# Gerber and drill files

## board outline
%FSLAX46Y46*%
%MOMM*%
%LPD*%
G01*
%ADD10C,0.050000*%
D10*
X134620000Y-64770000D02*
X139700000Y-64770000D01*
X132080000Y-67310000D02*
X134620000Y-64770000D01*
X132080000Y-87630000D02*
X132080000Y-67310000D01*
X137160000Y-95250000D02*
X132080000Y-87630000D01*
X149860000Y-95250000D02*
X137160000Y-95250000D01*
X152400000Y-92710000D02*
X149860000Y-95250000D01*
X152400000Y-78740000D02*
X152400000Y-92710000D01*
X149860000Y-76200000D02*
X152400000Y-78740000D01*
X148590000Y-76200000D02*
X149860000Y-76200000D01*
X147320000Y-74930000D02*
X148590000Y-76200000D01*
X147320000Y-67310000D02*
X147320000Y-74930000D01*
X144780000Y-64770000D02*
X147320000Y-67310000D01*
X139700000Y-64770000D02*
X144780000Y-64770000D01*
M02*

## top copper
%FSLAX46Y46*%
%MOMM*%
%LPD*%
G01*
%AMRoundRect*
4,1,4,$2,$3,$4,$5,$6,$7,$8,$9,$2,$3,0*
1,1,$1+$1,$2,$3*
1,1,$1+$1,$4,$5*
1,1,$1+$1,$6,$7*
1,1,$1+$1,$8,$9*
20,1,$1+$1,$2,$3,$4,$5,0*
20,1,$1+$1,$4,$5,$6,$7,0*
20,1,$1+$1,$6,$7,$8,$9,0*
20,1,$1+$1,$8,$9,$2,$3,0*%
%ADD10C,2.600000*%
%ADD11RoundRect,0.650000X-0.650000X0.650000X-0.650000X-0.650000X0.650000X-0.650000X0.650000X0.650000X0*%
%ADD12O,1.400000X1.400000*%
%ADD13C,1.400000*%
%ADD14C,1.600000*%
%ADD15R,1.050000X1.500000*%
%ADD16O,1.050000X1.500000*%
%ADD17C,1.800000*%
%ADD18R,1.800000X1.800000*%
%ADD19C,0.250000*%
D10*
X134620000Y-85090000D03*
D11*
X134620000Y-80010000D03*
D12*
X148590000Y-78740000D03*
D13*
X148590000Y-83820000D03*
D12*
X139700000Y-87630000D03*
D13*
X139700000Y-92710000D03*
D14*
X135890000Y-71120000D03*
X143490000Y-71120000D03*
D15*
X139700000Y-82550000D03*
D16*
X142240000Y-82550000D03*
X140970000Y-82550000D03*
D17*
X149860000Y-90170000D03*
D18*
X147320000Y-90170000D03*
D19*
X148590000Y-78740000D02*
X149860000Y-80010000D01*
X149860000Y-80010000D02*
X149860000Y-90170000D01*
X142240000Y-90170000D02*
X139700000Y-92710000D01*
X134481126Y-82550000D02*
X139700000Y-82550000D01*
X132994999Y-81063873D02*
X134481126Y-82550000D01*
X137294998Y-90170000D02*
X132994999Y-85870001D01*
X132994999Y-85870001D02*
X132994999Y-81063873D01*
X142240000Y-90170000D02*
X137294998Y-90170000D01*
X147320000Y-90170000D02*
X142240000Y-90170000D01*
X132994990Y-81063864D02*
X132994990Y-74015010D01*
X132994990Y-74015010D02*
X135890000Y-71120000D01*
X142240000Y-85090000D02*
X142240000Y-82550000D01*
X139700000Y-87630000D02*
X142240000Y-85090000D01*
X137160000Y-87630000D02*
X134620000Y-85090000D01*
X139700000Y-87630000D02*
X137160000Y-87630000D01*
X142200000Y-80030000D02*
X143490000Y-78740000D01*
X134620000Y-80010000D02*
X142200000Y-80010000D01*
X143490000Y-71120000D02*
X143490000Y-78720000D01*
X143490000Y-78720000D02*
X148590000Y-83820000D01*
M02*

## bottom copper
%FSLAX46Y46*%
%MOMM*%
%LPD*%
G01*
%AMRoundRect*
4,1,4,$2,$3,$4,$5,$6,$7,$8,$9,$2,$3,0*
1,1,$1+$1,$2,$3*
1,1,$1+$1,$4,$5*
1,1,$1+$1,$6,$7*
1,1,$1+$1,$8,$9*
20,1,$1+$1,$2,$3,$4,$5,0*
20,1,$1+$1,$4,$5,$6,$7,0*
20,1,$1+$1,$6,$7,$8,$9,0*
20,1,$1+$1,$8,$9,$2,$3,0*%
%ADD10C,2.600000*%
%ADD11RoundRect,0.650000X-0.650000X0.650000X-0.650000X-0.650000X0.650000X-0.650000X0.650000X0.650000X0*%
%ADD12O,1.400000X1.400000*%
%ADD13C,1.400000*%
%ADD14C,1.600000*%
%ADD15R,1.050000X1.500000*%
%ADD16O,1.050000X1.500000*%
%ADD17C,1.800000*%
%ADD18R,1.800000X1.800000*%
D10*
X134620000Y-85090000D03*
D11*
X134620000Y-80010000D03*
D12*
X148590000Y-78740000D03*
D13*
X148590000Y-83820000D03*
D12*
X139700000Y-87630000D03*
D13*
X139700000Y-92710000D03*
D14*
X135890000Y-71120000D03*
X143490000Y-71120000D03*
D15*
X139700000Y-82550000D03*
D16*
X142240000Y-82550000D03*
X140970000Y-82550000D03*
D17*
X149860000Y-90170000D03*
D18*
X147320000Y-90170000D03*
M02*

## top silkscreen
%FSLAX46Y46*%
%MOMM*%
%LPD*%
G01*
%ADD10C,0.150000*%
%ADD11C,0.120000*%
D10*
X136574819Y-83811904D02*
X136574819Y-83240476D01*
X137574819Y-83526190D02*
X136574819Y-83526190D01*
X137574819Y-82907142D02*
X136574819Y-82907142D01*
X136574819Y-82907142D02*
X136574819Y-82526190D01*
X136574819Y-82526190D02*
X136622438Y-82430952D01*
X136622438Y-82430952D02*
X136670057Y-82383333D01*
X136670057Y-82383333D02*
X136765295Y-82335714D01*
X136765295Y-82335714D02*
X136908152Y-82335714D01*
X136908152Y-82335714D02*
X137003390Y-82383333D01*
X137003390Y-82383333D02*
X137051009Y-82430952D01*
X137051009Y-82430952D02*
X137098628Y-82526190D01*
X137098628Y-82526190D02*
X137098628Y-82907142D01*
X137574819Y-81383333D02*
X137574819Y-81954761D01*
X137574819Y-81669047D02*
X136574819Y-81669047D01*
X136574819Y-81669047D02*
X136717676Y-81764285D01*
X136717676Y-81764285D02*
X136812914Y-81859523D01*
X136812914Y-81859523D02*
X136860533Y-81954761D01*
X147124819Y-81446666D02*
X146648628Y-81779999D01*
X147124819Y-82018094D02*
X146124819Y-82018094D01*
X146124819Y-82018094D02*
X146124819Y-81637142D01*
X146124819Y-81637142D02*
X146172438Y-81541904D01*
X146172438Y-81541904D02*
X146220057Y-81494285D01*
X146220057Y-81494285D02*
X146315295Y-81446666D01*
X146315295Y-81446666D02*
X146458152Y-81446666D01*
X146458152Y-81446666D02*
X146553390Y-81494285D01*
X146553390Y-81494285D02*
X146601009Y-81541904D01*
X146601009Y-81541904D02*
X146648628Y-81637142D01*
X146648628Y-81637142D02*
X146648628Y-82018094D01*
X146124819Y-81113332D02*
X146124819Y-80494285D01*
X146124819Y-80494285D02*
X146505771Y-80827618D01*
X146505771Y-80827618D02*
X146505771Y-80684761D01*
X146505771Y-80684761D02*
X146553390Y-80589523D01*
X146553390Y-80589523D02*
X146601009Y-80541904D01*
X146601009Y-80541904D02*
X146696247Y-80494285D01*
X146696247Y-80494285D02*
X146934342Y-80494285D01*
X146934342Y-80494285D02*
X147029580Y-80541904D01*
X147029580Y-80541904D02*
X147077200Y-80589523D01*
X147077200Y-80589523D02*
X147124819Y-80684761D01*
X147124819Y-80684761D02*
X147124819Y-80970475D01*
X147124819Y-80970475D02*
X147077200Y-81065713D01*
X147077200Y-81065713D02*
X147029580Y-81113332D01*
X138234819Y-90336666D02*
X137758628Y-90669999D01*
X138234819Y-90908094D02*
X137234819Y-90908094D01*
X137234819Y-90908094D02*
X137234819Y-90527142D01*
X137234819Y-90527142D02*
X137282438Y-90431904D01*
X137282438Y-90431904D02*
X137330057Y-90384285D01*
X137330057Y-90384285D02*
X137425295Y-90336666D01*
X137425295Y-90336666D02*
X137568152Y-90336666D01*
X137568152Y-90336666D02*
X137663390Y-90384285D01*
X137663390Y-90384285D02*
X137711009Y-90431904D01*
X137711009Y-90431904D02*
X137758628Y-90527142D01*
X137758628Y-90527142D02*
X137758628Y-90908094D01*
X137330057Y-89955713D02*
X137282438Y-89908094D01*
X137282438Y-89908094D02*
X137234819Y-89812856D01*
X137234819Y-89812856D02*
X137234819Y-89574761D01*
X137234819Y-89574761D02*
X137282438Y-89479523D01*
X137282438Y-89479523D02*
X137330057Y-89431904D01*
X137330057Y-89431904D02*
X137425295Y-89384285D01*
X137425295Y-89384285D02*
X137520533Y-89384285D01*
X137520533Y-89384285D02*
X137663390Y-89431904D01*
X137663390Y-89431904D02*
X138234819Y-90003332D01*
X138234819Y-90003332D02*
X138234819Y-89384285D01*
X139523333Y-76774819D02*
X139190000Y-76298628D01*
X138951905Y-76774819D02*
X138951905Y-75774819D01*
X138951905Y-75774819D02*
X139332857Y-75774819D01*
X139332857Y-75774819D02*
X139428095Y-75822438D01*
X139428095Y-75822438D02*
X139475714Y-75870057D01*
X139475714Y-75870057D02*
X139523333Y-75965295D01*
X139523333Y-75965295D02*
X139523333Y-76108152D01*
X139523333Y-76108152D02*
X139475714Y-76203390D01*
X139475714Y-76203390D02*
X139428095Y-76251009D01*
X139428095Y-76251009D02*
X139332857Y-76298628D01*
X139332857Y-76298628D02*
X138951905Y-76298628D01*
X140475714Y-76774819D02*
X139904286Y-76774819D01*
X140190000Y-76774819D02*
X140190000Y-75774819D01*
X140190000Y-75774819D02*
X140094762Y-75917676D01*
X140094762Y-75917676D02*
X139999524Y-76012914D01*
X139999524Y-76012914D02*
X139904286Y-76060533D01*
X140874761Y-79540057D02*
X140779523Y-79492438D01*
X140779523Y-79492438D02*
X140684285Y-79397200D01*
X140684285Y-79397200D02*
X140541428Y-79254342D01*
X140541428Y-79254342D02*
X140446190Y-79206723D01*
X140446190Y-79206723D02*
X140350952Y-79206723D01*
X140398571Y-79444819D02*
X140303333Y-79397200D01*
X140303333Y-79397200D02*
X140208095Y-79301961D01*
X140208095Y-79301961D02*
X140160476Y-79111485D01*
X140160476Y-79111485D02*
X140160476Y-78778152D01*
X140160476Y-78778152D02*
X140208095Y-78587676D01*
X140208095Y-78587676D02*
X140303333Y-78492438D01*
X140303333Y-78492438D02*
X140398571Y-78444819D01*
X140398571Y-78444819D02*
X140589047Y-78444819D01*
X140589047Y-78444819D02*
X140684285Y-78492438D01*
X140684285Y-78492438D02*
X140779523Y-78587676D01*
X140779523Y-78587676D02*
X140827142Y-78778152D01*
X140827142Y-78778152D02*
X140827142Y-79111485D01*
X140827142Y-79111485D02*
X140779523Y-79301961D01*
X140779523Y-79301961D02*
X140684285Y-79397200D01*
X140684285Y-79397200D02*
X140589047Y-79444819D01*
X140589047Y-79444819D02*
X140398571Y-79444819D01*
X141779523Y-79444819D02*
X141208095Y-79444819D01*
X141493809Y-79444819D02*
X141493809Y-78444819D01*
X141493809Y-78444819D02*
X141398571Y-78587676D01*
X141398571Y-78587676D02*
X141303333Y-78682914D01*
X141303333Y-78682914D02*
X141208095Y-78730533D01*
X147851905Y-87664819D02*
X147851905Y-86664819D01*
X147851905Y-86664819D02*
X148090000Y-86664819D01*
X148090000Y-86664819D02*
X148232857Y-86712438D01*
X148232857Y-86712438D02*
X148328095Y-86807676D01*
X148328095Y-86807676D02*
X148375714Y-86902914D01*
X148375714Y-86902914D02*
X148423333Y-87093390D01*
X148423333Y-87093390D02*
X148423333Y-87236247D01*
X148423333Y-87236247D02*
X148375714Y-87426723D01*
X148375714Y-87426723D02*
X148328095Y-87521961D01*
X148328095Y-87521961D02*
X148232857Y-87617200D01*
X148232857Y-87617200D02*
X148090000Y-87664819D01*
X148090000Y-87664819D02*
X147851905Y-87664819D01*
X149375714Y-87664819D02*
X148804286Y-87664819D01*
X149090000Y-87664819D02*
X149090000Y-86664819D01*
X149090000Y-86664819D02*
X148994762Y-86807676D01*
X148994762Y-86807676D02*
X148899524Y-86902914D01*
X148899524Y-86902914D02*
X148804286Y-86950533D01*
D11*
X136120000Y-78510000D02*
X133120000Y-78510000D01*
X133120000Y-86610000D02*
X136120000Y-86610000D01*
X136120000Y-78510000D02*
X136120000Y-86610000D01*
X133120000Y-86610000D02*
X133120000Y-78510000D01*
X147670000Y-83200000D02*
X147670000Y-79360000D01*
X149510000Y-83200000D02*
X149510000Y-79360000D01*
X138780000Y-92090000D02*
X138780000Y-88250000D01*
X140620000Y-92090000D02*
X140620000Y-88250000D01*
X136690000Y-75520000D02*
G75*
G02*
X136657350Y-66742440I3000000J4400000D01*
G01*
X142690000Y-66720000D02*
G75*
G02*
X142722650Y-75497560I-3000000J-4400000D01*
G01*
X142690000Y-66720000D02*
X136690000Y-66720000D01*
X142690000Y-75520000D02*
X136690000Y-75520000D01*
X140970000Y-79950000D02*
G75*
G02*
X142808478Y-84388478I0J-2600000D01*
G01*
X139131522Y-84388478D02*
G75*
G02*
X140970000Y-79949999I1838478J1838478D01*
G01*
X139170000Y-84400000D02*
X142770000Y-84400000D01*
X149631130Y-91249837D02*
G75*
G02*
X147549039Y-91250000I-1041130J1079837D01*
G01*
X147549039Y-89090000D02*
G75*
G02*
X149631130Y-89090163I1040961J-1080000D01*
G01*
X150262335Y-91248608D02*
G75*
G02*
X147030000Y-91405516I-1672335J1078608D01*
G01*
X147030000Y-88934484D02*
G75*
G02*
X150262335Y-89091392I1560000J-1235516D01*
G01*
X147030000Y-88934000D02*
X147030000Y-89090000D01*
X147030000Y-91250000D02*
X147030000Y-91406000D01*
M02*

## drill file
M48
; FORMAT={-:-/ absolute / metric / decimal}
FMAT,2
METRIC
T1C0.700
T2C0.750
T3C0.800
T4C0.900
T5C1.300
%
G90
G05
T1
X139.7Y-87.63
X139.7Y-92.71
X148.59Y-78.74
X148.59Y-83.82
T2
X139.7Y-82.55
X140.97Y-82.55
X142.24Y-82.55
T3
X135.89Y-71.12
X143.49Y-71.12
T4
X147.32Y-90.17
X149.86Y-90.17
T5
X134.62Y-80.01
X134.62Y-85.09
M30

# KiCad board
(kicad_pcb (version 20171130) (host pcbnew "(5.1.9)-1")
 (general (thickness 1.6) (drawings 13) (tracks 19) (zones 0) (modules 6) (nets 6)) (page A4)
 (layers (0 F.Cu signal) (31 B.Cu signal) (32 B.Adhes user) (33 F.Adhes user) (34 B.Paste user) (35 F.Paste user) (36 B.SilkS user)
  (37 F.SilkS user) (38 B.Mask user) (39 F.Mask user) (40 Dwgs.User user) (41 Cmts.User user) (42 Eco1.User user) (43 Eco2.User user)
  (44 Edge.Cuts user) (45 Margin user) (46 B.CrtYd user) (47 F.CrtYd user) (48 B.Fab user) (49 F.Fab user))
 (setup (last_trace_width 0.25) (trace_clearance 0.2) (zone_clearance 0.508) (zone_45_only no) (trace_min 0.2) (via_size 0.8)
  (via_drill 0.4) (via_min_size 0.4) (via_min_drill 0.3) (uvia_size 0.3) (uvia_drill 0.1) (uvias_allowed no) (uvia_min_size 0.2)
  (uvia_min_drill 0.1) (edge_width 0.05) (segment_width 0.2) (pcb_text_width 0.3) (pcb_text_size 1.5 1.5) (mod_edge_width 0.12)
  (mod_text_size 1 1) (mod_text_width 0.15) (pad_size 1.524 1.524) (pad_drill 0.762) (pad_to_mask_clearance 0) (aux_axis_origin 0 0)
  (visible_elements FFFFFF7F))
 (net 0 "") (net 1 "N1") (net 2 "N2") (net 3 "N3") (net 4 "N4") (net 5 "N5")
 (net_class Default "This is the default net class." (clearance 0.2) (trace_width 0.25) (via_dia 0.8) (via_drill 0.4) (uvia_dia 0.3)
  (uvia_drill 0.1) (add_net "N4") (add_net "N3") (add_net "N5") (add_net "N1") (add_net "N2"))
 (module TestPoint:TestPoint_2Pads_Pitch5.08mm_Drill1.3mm (layer F.Cu) (at 134.62 80.01 270)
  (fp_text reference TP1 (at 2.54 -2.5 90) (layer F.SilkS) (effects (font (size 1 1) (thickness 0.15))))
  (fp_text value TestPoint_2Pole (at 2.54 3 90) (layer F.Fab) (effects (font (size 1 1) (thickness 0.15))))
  (fp_line (start -1.5 -1.5) (end -1.5 1.5) (layer F.SilkS) (width 0.12))
  (fp_line (start 6.6 1.5) (end 6.6 -1.5) (layer F.SilkS) (width 0.12))
  (fp_line (start -1.5 -1.5) (end 6.6 -1.5) (layer F.SilkS) (width 0.12))
  (fp_line (start 6.6 1.5) (end -1.5 1.5) (layer F.SilkS) (width 0.12))
  (pad 2 thru_hole circle (at 5.08 0 270) (size 2.6 2.6) (drill 1.3) (layers *.Cu *.Mask) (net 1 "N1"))
  (pad 1 thru_hole roundrect (at 0 0 270) (size 2.6 2.6) (drill 1.3) (layers *.Cu *.Mask) (roundrect_rratio 0.25) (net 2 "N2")))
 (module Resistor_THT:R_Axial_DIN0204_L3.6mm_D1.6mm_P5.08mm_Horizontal (layer F.Cu) (at 148.59 83.82 90)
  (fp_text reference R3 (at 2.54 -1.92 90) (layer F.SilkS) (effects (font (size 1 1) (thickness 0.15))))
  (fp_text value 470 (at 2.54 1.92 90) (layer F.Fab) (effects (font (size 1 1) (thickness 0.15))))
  (fp_line (start 0.62 -0.92) (end 4.46 -0.92) (layer F.SilkS) (width 0.12))
  (fp_line (start 0.62 0.92) (end 4.46 0.92) (layer F.SilkS) (width 0.12))
  (pad 2 thru_hole oval (at 5.08 0 90) (size 1.4 1.4) (drill 0.7) (layers *.Cu *.Mask) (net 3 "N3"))
  (pad 1 thru_hole circle (at 0 0 90) (size 1.4 1.4) (drill 0.7) (layers *.Cu *.Mask) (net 2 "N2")))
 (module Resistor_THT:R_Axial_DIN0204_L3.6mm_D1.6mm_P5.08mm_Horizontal (layer F.Cu) (at 139.7 92.71 90)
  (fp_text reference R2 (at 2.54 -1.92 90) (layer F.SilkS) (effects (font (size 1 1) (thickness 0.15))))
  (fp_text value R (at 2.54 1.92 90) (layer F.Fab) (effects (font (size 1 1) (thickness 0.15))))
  (fp_line (start 0.62 -0.92) (end 4.46 -0.92) (layer F.SilkS) (width 0.12))
  (fp_line (start 0.62 0.92) (end 4.46 0.92) (layer F.SilkS) (width 0.12))
  (pad 2 thru_hole oval (at 5.08 0 90) (size 1.4 1.4) (drill 0.7) (layers *.Cu *.Mask) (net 1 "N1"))
  (pad 1 thru_hole circle (at 0 0 90) (size 1.4 1.4) (drill 0.7) (layers *.Cu *.Mask) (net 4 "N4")))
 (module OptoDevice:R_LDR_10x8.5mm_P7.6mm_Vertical (layer F.Cu) (at 143.49 71.12 180)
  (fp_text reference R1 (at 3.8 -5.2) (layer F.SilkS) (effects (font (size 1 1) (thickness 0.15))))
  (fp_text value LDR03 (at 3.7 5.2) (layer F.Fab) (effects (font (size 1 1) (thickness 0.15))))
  (fp_arc (start 3.8 0) (end 6.8 -4.4) (angle 111) (layer F.SilkS) (width 0.12))
  (fp_arc (start 3.8 0) (end 0.8 4.4) (angle 111) (layer F.SilkS) (width 0.12))
  (fp_line (start 0.8 4.4) (end 6.8 4.4) (layer F.SilkS) (width 0.12))
  (fp_line (start 0.8 -4.4) (end 6.8 -4.4) (layer F.SilkS) (width 0.12))
  (pad 2 thru_hole circle (at 7.6 0 180) (size 1.6 1.6) (drill 0.8) (layers *.Cu *.Mask) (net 4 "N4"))
  (pad 1 thru_hole circle (at 0 0 180) (size 1.6 1.6) (drill 0.8) (layers *.Cu *.Mask) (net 2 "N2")))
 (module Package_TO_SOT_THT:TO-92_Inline (layer F.Cu) (at 139.7 82.55)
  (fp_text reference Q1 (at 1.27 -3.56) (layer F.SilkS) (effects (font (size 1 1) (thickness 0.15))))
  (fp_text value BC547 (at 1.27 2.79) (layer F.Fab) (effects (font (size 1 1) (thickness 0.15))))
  (fp_arc (start 1.27 0) (end 1.27 -2.6) (angle 135) (layer F.SilkS) (width 0.12))
  (fp_arc (start 1.27 0) (end 1.27 -2.6) (angle -135) (layer F.SilkS) (width 0.12))
  (fp_line (start -0.53 1.85) (end 3.07 1.85) (layer F.SilkS) (width 0.12))
  (pad 1 thru_hole rect (at 0 0) (size 1.05 1.5) (drill 0.75) (layers *.Cu *.Mask) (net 4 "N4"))
  (pad 3 thru_hole oval (at 2.54 0) (size 1.05 1.5) (drill 0.75) (layers *.Cu *.Mask) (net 1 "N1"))
  (pad 2 thru_hole oval (at 1.27 0) (size 1.05 1.5) (drill 0.75) (layers *.Cu *.Mask) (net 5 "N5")))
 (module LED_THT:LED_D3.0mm (layer F.Cu) (at 147.32 90.17)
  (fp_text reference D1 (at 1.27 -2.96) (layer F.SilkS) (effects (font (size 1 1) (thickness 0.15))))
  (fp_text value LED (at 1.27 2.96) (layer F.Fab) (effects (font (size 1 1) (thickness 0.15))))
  (fp_arc (start 1.27 0) (end 0.229039 1.08) (angle -87.9) (layer F.SilkS) (width 0.12))
  (fp_arc (start 1.27 0) (end 0.229039 -1.08) (angle 87.9) (layer F.SilkS) (width 0.12))
  (fp_arc (start 1.27 0) (end -0.29 1.235516) (angle -108.8) (layer F.SilkS) (width 0.12))
  (fp_arc (start 1.27 0) (end -0.29 -1.235516) (angle 108.8) (layer F.SilkS) (width 0.12))
  (fp_line (start -0.29 -1.236) (end -0.29 -1.08) (layer F.SilkS) (width 0.12))
  (fp_line (start -0.29 1.08) (end -0.29 1.236) (layer F.SilkS) (width 0.12))
  (pad 2 thru_hole circle (at 2.54 0) (size 1.8 1.8) (drill 0.9) (layers *.Cu *.Mask) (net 3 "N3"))
  (pad 1 thru_hole rect (at 0 0) (size 1.8 1.8) (drill 0.9) (layers *.Cu *.Mask) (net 4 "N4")))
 (gr_line (start 134.62 64.77) (end 139.7 64.77) (layer Edge.Cuts) (width 0.05))
 (gr_line (start 132.08 67.31) (end 134.62 64.77) (layer Edge.Cuts) (width 0.05))
 (gr_line (start 132.08 87.63) (end 132.08 67.31) (layer Edge.Cuts) (width 0.05))
 (gr_line (start 137.16 95.25) (end 132.08 87.63) (layer Edge.Cuts) (width 0.05))
 (gr_line (start 149.86 95.25) (end 137.16 95.25) (layer Edge.Cuts) (width 0.05))
 (gr_line (start 152.4 92.71) (end 149.86 95.25) (layer Edge.Cuts) (width 0.05))
 (gr_line (start 152.4 78.74) (end 152.4 92.71) (layer Edge.Cuts) (width 0.05))
 (gr_line (start 149.86 76.2) (end 152.4 78.74) (layer Edge.Cuts) (width 0.05))
 (gr_line (start 148.59 76.2) (end 149.86 76.2) (layer Edge.Cuts) (width 0.05))
 (gr_line (start 147.32 74.93) (end 148.59 76.2) (layer Edge.Cuts) (width 0.05))
 (gr_line (start 147.32 67.31) (end 147.32 74.93) (layer Edge.Cuts) (width 0.05))
 (gr_line (start 144.78 64.77) (end 147.32 67.31) (layer Edge.Cuts) (width 0.05))
 (gr_line (start 139.7 64.77) (end 144.78 64.77) (layer Edge.Cuts) (width 0.05))
 (segment (start 148.59 78.74) (end 149.86 80.01) (width 0.25) (layer F.Cu) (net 3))
 (segment (start 149.86 80.01) (end 149.86 90.17) (width 0.25) (layer F.Cu) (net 3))
 (segment (start 142.24 90.17) (end 139.7 92.71) (width 0.25) (layer F.Cu) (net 4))
 (segment (start 134.481126 82.55) (end 139.7 82.55) (width 0.25) (layer F.Cu) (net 4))
 (segment (start 132.994999 81.063873) (end 134.481126 82.55) (width 0.25) (layer F.Cu) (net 4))
 (segment (start 137.294998 90.17) (end 132.994999 85.870001) (width 0.25) (layer F.Cu) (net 4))
 (segment (start 132.994999 85.870001) (end 132.994999 81.063873) (width 0.25) (layer F.Cu) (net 4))
 (segment (start 142.24 90.17) (end 137.294998 90.17) (width 0.25) (layer F.Cu) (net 4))
 (segment (start 147.32 90.17) (end 142.24 90.17) (width 0.25) (layer F.Cu) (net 4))
 (segment (start 132.99499 81.063864) (end 132.99499 74.01501) (width 0.25) (layer F.Cu) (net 4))
 (segment (start 132.99499 74.01501) (end 135.89 71.12) (width 0.25) (layer F.Cu) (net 4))
 (segment (start 142.24 85.09) (end 142.24 82.55) (width 0.25) (layer F.Cu) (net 1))
 (segment (start 139.7 87.63) (end 142.24 85.09) (width 0.25) (layer F.Cu) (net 1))
 (segment (start 137.16 87.63) (end 134.62 85.09) (width 0.25) (layer F.Cu) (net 1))
 (segment (start 139.7 87.63) (end 137.16 87.63) (width 0.25) (layer F.Cu) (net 1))
 (segment (start 142.2 80.03) (end 143.49 78.74) (width 0.25) (layer F.Cu) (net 2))
 (segment (start 134.62 80.01) (end 142.2 80.01) (width 0.25) (layer F.Cu) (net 2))
 (segment (start 143.49 71.12) (end 143.49 78.72) (width 0.25) (layer F.Cu) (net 2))
 (segment (start 143.49 78.72) (end 148.59 83.82) (width 0.25) (layer F.Cu) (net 2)))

